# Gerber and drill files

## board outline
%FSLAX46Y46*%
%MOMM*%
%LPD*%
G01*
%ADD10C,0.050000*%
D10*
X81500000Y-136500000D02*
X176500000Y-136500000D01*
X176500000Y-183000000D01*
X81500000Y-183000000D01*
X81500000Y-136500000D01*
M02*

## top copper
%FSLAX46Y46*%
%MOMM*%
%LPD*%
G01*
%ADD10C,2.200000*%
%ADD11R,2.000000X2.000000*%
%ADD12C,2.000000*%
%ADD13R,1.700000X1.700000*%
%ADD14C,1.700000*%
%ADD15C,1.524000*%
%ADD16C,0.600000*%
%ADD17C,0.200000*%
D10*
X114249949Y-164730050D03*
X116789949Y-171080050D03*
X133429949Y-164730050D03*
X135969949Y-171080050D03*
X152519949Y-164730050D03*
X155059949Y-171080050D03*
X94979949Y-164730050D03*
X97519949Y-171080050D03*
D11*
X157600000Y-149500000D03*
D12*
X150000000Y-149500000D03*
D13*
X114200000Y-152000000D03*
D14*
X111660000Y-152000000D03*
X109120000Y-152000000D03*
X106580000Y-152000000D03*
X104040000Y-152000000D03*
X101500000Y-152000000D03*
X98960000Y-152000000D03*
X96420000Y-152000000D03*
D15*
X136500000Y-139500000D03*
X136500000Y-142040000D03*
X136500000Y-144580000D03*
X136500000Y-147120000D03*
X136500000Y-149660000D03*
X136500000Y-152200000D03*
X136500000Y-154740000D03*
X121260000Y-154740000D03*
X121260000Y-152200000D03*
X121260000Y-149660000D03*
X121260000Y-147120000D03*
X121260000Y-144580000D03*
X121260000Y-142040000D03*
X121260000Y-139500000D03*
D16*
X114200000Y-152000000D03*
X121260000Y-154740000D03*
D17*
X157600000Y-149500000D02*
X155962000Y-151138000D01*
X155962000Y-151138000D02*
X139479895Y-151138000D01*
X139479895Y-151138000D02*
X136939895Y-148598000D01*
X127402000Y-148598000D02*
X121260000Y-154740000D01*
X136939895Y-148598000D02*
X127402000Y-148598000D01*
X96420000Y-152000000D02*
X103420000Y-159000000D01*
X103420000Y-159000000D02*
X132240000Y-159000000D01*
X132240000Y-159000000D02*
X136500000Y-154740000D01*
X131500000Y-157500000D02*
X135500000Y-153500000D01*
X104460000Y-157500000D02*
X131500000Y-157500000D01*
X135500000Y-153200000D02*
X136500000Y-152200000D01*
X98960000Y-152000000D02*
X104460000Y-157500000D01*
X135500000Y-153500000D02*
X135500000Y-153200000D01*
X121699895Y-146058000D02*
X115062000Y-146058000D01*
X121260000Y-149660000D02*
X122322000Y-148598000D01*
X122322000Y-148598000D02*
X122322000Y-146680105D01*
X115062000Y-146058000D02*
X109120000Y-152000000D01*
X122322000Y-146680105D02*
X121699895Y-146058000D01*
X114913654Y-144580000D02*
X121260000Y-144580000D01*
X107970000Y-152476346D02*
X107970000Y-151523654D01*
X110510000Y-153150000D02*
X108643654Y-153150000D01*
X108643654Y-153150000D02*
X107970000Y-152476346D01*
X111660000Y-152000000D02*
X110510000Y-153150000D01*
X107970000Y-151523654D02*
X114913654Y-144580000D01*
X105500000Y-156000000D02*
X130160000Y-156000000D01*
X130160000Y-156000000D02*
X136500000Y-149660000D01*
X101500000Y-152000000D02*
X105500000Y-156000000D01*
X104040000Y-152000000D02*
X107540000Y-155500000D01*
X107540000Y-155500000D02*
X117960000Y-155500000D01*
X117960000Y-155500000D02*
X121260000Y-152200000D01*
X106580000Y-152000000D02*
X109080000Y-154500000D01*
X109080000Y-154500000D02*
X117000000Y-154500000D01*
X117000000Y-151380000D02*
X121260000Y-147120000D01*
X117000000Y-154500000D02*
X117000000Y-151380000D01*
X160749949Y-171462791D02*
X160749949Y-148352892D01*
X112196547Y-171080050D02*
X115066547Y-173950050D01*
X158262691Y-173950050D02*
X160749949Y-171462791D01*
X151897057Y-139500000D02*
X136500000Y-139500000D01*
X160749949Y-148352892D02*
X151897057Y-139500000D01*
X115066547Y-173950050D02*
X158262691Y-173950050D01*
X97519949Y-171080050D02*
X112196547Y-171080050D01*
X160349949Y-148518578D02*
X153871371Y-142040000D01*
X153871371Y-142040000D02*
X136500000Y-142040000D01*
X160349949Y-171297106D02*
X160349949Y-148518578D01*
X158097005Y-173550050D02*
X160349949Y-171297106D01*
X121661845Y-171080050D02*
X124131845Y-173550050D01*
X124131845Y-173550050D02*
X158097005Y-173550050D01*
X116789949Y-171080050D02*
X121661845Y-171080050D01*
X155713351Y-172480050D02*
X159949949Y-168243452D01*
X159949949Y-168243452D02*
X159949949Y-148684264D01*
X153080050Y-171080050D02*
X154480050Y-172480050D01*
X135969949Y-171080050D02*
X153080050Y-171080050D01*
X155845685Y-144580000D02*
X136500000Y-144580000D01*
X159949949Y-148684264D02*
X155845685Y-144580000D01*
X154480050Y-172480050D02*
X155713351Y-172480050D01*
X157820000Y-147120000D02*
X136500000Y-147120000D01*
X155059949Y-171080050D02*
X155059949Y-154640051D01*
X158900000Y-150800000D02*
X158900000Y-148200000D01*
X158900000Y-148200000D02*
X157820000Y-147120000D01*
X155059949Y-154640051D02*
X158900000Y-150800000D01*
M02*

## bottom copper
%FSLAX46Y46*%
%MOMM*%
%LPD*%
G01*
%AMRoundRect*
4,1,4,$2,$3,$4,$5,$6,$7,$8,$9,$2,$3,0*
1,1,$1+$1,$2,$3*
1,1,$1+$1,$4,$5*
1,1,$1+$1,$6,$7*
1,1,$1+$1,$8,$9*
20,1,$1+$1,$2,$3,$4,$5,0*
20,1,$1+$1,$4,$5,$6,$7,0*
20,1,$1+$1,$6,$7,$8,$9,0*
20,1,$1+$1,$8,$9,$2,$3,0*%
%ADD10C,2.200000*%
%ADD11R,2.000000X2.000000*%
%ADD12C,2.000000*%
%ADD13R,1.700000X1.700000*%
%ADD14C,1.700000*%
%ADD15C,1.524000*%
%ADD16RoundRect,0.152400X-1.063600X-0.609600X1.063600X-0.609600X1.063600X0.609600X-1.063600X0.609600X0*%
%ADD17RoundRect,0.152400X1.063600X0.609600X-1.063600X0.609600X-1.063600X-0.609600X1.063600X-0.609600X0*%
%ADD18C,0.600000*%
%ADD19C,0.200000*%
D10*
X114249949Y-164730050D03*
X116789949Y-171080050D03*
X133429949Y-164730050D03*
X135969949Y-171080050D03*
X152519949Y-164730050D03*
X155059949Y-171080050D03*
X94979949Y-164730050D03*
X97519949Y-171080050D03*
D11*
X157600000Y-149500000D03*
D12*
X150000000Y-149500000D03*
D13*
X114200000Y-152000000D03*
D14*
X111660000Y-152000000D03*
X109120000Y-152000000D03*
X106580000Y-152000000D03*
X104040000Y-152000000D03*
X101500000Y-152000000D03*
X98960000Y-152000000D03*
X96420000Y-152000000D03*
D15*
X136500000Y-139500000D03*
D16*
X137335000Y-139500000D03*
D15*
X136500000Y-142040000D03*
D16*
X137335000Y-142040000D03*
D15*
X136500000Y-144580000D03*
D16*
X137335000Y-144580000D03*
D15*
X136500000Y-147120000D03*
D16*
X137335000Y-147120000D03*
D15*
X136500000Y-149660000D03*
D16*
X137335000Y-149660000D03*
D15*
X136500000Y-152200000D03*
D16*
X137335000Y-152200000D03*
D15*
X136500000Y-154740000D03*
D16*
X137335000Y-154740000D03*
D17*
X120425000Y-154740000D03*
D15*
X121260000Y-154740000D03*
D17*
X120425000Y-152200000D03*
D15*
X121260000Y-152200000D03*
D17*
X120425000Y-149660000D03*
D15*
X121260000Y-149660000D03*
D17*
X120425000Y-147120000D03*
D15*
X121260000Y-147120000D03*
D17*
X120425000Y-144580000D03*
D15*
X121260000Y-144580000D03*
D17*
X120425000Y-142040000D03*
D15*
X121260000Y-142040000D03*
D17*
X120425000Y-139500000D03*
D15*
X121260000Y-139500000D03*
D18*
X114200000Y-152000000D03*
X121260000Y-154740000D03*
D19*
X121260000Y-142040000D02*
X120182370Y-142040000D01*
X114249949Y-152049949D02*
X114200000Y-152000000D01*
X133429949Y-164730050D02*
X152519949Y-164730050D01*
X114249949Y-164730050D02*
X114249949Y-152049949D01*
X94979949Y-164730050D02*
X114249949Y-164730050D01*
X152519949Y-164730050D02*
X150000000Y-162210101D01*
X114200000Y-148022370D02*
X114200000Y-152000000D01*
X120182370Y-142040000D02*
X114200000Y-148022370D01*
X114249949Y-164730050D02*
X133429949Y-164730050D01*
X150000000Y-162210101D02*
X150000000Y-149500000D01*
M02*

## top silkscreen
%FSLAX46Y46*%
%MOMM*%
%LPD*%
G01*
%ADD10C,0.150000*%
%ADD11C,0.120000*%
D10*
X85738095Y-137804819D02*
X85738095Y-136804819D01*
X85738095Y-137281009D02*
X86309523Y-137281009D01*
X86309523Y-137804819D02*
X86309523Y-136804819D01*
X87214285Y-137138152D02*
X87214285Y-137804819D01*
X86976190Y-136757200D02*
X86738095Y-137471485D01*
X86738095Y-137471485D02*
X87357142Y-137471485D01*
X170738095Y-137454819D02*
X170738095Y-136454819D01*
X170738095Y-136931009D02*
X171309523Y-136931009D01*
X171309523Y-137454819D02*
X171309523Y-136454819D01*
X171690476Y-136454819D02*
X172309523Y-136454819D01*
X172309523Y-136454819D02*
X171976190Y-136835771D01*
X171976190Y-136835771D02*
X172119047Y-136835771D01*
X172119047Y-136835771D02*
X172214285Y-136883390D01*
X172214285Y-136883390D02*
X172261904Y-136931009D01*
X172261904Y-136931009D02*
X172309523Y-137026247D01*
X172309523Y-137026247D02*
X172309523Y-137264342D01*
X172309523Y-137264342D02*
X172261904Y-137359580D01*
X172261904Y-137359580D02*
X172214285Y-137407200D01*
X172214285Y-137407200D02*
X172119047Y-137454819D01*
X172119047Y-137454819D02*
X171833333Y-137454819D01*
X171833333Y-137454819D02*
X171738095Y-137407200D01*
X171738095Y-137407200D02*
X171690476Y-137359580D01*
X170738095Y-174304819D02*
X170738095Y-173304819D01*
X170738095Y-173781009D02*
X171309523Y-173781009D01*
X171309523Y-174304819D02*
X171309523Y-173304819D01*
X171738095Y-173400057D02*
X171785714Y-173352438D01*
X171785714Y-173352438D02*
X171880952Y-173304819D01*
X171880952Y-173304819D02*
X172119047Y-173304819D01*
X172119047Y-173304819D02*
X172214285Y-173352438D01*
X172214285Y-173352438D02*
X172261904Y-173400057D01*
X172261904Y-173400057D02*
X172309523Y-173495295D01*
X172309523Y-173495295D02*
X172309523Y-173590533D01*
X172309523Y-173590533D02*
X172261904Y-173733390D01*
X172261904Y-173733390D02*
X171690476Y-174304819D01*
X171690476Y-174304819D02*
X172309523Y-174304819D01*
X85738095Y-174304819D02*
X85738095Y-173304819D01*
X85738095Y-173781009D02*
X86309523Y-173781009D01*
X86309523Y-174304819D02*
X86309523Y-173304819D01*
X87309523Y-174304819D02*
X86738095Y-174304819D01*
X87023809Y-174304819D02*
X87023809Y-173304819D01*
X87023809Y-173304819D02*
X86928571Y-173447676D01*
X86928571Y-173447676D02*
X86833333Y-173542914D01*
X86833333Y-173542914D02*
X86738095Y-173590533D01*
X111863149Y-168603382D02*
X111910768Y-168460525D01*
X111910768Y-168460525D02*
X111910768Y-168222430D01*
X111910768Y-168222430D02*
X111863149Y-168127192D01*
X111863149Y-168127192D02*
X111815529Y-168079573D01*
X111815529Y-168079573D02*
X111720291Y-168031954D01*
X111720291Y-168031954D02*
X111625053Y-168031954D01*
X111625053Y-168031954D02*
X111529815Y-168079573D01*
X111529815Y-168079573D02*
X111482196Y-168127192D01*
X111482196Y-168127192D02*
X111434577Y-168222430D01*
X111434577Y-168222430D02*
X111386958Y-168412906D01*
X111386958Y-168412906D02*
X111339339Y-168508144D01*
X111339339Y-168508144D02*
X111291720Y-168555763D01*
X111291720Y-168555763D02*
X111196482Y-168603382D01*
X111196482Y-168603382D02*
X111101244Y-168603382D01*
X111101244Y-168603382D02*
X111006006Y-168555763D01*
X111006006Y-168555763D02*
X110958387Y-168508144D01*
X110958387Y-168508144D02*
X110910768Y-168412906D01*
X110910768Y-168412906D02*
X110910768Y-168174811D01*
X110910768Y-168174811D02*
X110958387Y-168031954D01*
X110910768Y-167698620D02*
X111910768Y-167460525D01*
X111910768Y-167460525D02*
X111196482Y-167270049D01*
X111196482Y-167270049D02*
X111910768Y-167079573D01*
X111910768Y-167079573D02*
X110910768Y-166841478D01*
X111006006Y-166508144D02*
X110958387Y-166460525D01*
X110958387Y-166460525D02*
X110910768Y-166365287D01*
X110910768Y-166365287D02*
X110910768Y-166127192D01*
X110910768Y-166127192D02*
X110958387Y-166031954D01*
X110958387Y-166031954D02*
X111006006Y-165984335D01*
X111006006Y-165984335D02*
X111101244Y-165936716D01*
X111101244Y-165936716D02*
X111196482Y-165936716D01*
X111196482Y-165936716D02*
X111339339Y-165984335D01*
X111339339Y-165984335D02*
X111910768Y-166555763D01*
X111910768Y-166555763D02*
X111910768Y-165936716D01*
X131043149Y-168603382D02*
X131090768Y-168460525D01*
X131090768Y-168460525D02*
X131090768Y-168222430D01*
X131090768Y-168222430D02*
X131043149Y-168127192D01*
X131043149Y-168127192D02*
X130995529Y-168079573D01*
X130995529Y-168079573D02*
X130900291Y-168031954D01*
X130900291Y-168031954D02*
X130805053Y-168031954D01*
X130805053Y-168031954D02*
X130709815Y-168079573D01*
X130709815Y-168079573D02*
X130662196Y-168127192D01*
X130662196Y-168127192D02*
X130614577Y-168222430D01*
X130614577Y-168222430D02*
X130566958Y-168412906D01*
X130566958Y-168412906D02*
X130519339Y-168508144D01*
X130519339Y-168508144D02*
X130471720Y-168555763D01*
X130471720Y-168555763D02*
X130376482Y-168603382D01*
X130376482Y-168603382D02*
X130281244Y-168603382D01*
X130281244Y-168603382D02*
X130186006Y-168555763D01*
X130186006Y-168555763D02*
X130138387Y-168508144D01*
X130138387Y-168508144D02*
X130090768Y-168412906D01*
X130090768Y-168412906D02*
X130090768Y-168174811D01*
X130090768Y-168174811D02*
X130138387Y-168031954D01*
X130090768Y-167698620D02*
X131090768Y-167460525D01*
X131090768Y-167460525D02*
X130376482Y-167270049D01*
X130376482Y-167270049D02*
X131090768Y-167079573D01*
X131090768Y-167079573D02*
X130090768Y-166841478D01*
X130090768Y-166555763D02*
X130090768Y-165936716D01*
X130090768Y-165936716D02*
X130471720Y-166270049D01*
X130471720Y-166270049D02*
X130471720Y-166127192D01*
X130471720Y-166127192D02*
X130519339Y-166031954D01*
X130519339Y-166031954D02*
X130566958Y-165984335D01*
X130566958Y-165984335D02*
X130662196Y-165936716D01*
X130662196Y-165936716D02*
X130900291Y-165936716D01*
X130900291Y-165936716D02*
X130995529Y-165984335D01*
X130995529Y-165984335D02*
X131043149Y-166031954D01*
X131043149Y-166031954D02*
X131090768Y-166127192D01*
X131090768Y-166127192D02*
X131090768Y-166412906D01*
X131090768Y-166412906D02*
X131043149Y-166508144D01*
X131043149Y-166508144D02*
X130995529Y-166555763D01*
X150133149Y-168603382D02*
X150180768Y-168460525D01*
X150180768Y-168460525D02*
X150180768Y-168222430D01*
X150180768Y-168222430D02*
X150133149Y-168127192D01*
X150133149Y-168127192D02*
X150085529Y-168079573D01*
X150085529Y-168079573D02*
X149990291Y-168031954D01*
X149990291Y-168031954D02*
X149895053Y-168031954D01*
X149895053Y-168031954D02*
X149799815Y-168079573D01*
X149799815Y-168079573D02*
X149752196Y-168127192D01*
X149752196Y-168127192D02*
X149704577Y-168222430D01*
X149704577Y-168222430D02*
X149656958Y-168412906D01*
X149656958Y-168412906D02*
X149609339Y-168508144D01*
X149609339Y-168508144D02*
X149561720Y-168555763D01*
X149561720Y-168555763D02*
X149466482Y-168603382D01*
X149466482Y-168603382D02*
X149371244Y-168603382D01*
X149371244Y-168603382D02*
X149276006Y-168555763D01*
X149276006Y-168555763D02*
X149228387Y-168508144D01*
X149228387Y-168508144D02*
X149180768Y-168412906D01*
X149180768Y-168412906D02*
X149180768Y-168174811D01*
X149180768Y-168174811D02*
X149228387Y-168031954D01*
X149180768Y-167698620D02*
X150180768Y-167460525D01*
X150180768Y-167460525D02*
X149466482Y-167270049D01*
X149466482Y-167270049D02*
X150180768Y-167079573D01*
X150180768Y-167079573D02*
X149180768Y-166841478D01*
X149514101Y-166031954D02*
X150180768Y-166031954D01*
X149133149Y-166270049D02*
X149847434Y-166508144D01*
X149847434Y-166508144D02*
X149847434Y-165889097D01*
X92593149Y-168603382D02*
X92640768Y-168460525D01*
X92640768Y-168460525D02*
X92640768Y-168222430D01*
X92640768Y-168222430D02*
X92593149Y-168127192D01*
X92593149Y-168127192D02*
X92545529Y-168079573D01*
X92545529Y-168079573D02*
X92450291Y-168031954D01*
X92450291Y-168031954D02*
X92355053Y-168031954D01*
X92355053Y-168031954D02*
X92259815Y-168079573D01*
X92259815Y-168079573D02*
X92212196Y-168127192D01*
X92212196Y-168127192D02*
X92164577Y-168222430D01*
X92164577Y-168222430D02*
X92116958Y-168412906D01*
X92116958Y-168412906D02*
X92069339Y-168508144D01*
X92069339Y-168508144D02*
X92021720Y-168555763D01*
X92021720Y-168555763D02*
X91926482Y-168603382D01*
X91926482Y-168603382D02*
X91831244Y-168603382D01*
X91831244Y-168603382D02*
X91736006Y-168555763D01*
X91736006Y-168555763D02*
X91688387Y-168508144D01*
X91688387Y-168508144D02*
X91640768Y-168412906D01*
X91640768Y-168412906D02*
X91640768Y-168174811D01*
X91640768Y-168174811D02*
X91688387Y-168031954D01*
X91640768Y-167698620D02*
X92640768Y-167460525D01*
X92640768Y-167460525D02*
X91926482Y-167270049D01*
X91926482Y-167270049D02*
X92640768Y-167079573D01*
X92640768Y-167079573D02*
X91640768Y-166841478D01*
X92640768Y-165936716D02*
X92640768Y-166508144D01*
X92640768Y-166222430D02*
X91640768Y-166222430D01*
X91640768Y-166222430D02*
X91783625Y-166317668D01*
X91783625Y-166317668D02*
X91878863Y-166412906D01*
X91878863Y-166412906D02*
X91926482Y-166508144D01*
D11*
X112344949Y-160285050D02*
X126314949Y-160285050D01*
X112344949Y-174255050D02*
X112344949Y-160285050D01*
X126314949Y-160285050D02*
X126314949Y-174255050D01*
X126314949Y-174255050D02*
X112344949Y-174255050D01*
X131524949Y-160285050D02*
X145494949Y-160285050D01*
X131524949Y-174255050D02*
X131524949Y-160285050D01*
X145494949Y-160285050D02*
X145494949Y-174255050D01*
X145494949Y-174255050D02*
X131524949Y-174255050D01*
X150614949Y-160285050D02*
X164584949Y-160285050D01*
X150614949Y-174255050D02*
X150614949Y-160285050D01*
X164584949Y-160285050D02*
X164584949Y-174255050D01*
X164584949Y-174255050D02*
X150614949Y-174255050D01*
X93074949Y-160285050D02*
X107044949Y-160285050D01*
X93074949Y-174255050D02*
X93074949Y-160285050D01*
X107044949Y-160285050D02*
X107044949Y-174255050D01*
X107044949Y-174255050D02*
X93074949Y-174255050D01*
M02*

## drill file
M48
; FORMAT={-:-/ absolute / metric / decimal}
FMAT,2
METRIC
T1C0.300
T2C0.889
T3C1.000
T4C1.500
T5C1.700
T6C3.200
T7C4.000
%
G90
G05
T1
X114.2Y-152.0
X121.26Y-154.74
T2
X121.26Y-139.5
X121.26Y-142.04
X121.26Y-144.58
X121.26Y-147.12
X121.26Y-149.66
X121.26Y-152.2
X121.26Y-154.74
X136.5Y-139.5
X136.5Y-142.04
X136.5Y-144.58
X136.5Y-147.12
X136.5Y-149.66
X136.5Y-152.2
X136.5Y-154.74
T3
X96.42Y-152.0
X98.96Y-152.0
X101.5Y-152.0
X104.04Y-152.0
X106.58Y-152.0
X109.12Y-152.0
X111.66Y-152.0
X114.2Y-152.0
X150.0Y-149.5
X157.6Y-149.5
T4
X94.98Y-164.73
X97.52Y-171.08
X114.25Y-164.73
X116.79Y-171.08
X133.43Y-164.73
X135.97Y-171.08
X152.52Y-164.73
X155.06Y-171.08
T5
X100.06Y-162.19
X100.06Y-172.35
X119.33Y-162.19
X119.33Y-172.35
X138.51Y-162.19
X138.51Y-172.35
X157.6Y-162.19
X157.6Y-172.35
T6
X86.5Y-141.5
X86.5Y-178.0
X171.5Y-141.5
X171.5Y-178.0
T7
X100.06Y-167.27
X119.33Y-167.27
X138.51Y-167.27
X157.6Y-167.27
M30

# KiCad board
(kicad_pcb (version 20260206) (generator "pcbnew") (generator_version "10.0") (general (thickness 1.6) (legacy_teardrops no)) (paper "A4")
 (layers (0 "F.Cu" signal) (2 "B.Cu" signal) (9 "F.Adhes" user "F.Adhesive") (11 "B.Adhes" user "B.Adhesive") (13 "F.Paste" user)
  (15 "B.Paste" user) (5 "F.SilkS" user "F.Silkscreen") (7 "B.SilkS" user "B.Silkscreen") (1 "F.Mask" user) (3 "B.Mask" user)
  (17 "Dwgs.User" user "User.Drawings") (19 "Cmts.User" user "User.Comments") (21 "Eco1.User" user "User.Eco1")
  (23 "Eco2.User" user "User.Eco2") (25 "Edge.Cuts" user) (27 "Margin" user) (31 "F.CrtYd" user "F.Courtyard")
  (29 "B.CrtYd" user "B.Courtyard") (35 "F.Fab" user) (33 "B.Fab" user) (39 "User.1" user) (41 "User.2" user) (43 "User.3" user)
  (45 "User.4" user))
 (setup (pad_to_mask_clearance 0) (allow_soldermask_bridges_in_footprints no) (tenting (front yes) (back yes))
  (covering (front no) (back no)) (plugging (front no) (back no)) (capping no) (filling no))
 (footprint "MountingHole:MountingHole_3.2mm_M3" (layer "F.Cu") (at 86.5 141.5)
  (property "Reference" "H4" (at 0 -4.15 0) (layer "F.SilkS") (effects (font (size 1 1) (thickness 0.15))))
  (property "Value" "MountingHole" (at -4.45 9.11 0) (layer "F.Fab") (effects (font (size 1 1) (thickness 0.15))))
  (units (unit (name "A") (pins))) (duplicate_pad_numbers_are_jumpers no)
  (pad "" np_thru_hole circle (at 0 0) (size 3.2 3.2) (drill 3.2) (layers "*.Cu" "*.Mask")))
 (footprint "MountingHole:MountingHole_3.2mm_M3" (layer "F.Cu") (at 171.5 141.5)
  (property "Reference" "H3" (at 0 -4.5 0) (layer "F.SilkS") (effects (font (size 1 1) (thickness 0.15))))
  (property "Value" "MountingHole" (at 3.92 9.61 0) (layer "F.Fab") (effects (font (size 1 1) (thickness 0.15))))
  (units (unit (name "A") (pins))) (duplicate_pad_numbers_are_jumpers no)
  (pad "" np_thru_hole circle (at 0 0) (size 3.2 3.2) (drill 3.2) (layers "*.Cu" "*.Mask")))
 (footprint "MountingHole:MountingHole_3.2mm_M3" (layer "F.Cu") (at 171.5 178)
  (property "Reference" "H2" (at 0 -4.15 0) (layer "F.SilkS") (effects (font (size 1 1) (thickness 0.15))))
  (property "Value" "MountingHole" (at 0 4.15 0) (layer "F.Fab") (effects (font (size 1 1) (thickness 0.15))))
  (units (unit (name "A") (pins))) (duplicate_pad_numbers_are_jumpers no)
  (pad "" np_thru_hole circle (at 0 0) (size 3.2 3.2) (drill 3.2) (layers "*.Cu" "*.Mask")))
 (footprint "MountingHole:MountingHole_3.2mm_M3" (layer "F.Cu") (at 86.5 178)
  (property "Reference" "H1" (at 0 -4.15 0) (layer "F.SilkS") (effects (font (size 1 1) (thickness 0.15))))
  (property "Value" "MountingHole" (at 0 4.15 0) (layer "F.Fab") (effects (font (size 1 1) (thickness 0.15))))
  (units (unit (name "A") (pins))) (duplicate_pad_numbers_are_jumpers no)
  (pad "" np_thru_hole circle (at 0 0) (size 3.2 3.2) (drill 3.2) (layers "*.Cu" "*.Mask")))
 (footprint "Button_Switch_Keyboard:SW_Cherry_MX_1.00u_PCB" (layer "F.Cu") (at 114.249949 164.73005 90)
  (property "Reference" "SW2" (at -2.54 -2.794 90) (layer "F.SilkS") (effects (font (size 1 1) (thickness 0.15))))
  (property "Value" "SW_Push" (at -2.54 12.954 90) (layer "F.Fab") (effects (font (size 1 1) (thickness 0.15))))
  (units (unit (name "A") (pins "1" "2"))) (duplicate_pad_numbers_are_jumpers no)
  (fp_line (start 4.445 -1.905) (end 4.445 12.065) (stroke (width 0.12) (type solid)) (layer "F.SilkS"))
  (fp_line (start -9.525 -1.905) (end 4.445 -1.905) (stroke (width 0.12) (type solid)) (layer "F.SilkS"))
  (fp_line (start 4.445 12.065) (end -9.525 12.065) (stroke (width 0.12) (type solid)) (layer "F.SilkS"))
  (fp_line (start -9.525 12.065) (end -9.525 -1.905) (stroke (width 0.12) (type solid)) (layer "F.SilkS"))
  (pad "" np_thru_hole circle (at -7.62 5.08 90) (size 1.7 1.7) (drill 1.7) (layers "*.Cu" "*.Mask"))
  (pad "" np_thru_hole circle (at -2.54 5.08 90) (size 4 4) (drill 4) (layers "*.Cu" "*.Mask"))
  (pad "" np_thru_hole circle (at 2.54 5.08 90) (size 1.7 1.7) (drill 1.7) (layers "*.Cu" "*.Mask"))
  (pad "1" thru_hole circle (at 0 0 90) (size 2.2 2.2) (drill 1.5) (layers "*.Cu" "*.Mask") (remove_unused_layers no) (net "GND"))
  (pad "2" thru_hole circle (at -6.35 2.54 90) (size 2.2 2.2) (drill 1.5) (layers "*.Cu" "*.Mask") (remove_unused_layers no)
   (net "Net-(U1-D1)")))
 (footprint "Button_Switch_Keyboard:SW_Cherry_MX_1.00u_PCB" (layer "F.Cu") (at 133.429949 164.73005 90)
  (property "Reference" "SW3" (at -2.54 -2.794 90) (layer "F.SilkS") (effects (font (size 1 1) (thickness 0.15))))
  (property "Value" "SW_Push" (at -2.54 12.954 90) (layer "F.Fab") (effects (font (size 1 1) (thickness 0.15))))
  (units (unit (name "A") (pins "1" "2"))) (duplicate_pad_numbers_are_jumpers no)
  (fp_line (start 4.445 -1.905) (end 4.445 12.065) (stroke (width 0.12) (type solid)) (layer "F.SilkS"))
  (fp_line (start -9.525 -1.905) (end 4.445 -1.905) (stroke (width 0.12) (type solid)) (layer "F.SilkS"))
  (fp_line (start 4.445 12.065) (end -9.525 12.065) (stroke (width 0.12) (type solid)) (layer "F.SilkS"))
  (fp_line (start -9.525 12.065) (end -9.525 -1.905) (stroke (width 0.12) (type solid)) (layer "F.SilkS"))
  (pad "" np_thru_hole circle (at -7.62 5.08 90) (size 1.7 1.7) (drill 1.7) (layers "*.Cu" "*.Mask"))
  (pad "" np_thru_hole circle (at -2.54 5.08 90) (size 4 4) (drill 4) (layers "*.Cu" "*.Mask"))
  (pad "" np_thru_hole circle (at 2.54 5.08 90) (size 1.7 1.7) (drill 1.7) (layers "*.Cu" "*.Mask"))
  (pad "1" thru_hole circle (at 0 0 90) (size 2.2 2.2) (drill 1.5) (layers "*.Cu" "*.Mask") (remove_unused_layers no) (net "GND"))
  (pad "2" thru_hole circle (at -6.35 2.54 90) (size 2.2 2.2) (drill 1.5) (layers "*.Cu" "*.Mask") (remove_unused_layers no)
   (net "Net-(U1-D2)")))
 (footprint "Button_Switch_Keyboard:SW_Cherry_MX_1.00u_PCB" (layer "F.Cu") (at 152.519949 164.73005 90)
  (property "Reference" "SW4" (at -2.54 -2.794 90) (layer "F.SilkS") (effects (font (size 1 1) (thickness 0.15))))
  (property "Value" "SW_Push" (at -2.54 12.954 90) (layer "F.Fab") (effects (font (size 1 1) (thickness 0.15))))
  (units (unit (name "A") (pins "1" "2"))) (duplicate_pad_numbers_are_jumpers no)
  (fp_line (start 4.445 -1.905) (end 4.445 12.065) (stroke (width 0.12) (type solid)) (layer "F.SilkS"))
  (fp_line (start -9.525 -1.905) (end 4.445 -1.905) (stroke (width 0.12) (type solid)) (layer "F.SilkS"))
  (fp_line (start 4.445 12.065) (end -9.525 12.065) (stroke (width 0.12) (type solid)) (layer "F.SilkS"))
  (fp_line (start -9.525 12.065) (end -9.525 -1.905) (stroke (width 0.12) (type solid)) (layer "F.SilkS"))
  (pad "" np_thru_hole circle (at -7.62 5.08 90) (size 1.7 1.7) (drill 1.7) (layers "*.Cu" "*.Mask"))
  (pad "" np_thru_hole circle (at -2.54 5.08 90) (size 4 4) (drill 4) (layers "*.Cu" "*.Mask"))
  (pad "" np_thru_hole circle (at 2.54 5.08 90) (size 1.7 1.7) (drill 1.7) (layers "*.Cu" "*.Mask"))
  (pad "1" thru_hole circle (at 0 0 90) (size 2.2 2.2) (drill 1.5) (layers "*.Cu" "*.Mask") (remove_unused_layers no) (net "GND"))
  (pad "2" thru_hole circle (at -6.35 2.54 90) (size 2.2 2.2) (drill 1.5) (layers "*.Cu" "*.Mask") (remove_unused_layers no)
   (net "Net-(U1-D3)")))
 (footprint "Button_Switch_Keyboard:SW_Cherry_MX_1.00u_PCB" (layer "F.Cu") (at 94.979949 164.73005 90)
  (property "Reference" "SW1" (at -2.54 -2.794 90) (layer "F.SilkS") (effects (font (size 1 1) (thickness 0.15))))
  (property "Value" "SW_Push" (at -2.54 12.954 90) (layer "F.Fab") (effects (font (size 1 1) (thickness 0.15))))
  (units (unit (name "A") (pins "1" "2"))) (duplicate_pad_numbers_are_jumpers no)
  (fp_line (start 4.445 -1.905) (end 4.445 12.065) (stroke (width 0.12) (type solid)) (layer "F.SilkS"))
  (fp_line (start -9.525 -1.905) (end 4.445 -1.905) (stroke (width 0.12) (type solid)) (layer "F.SilkS"))
  (fp_line (start 4.445 12.065) (end -9.525 12.065) (stroke (width 0.12) (type solid)) (layer "F.SilkS"))
  (fp_line (start -9.525 12.065) (end -9.525 -1.905) (stroke (width 0.12) (type solid)) (layer "F.SilkS"))
  (pad "" np_thru_hole circle (at -7.62 5.08 90) (size 1.7 1.7) (drill 1.7) (layers "*.Cu" "*.Mask"))
  (pad "" np_thru_hole circle (at -2.54 5.08 90) (size 4 4) (drill 4) (layers "*.Cu" "*.Mask"))
  (pad "" np_thru_hole circle (at 2.54 5.08 90) (size 1.7 1.7) (drill 1.7) (layers "*.Cu" "*.Mask"))
  (pad "1" thru_hole circle (at 0 0 90) (size 2.2 2.2) (drill 1.5) (layers "*.Cu" "*.Mask") (remove_unused_layers no) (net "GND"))
  (pad "2" thru_hole circle (at -6.35 2.54 90) (size 2.2 2.2) (drill 1.5) (layers "*.Cu" "*.Mask") (remove_unused_layers no)
   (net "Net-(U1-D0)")))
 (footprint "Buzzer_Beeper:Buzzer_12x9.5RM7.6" (layer "B.Cu") (at 157.6 149.5 180)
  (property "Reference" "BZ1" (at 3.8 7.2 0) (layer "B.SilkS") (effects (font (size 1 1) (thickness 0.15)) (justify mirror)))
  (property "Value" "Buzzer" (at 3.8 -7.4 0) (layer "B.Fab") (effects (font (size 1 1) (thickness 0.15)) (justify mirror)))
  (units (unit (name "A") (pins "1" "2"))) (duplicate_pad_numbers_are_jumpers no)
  (pad "1" thru_hole rect (at 0 0 180) (size 2 2) (drill 1) (layers "*.Cu" "*.Mask") (remove_unused_layers no) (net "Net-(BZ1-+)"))
  (pad "2" thru_hole circle (at 7.6 0 180) (size 2 2) (drill 1) (layers "*.Cu" "*.Mask") (remove_unused_layers no) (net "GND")))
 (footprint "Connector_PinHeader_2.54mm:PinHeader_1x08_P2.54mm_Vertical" (layer "B.Cu") (at 114.2 152 90)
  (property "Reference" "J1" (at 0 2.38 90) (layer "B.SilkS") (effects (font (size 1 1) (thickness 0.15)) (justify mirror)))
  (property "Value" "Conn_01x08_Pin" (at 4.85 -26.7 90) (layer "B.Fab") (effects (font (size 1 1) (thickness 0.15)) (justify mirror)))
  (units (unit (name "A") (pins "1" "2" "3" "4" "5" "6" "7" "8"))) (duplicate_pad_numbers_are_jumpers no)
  (pad "1" thru_hole rect (at 0 0 90) (size 1.7 1.7) (drill 1) (layers "*.Cu" "*.Mask") (remove_unused_layers no) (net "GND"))
  (pad "2" thru_hole circle (at 0 -2.54 90) (size 1.7 1.7) (drill 1) (layers "*.Cu" "*.Mask") (remove_unused_layers no) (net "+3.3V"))
  (pad "3" thru_hole circle (at 0 -5.08 90) (size 1.7 1.7) (drill 1) (layers "*.Cu" "*.Mask") (remove_unused_layers no) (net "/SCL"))
  (pad "4" thru_hole circle (at 0 -7.62 90) (size 1.7 1.7) (drill 1) (layers "*.Cu" "*.Mask") (remove_unused_layers no) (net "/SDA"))
  (pad "5" thru_hole circle (at 0 -10.16 90) (size 1.7 1.7) (drill 1) (layers "*.Cu" "*.Mask") (remove_unused_layers no) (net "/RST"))
  (pad "6" thru_hole circle (at 0 -12.7 90) (size 1.7 1.7) (drill 1) (layers "*.Cu" "*.Mask") (remove_unused_layers no) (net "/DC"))
  (pad "7" thru_hole circle (at 0 -15.24 90) (size 1.7 1.7) (drill 1) (layers "*.Cu" "*.Mask") (remove_unused_layers no) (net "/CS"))
  (pad "8" thru_hole circle (at 0 -17.78 90) (size 1.7 1.7) (drill 1) (layers "*.Cu" "*.Mask") (remove_unused_layers no) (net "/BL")))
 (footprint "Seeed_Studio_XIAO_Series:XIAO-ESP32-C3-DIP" (layer "B.Cu") (at 128.88 147.12 90)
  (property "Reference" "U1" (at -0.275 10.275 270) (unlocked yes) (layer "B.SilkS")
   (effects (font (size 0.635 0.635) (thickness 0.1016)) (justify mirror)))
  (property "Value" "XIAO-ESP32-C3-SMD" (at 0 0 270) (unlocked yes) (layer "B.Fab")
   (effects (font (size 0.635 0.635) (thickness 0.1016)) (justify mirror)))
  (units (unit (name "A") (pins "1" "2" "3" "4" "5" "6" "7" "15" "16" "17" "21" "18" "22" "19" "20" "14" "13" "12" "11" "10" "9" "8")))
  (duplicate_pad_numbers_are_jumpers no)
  (pad "1" thru_hole circle (at 7.62 7.62) (size 1.524 1.524) (drill 0.889) (layers "*.Cu" "*.Mask") (remove_unused_layers no)
   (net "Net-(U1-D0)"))
  (pad "1" smd roundrect (at 7.62 8.455) (size 2.432 1.524) (layers "B.Cu" "B.Mask") (roundrect_rratio 0.1) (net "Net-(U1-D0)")
   (thermal_bridge_angle 45))
  (pad "2" thru_hole circle (at 5.08 7.62) (size 1.524 1.524) (drill 0.889) (layers "*.Cu" "*.Mask") (remove_unused_layers no)
   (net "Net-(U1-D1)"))
  (pad "2" smd roundrect (at 5.08 8.455) (size 2.432 1.524) (layers "B.Cu" "B.Mask") (roundrect_rratio 0.1) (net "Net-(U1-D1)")
   (thermal_bridge_angle 45))
  (pad "3" thru_hole circle (at 2.54 7.62) (size 1.524 1.524) (drill 0.889) (layers "*.Cu" "*.Mask") (remove_unused_layers no)
   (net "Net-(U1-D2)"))
  (pad "3" smd roundrect (at 2.54 8.455) (size 2.432 1.524) (layers "B.Cu" "B.Mask") (roundrect_rratio 0.1) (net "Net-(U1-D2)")
   (thermal_bridge_angle 45))
  (pad "4" thru_hole circle (at 0 7.62) (size 1.524 1.524) (drill 0.889) (layers "*.Cu" "*.Mask") (remove_unused_layers no)
   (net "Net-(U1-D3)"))
  (pad "4" smd roundrect (at 0 8.455) (size 2.432 1.524) (layers "B.Cu" "B.Mask") (roundrect_rratio 0.1) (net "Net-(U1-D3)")
   (thermal_bridge_angle 45))
  (pad "5" thru_hole circle (at -2.54 7.62) (size 1.524 1.524) (drill 0.889) (layers "*.Cu" "*.Mask") (remove_unused_layers no) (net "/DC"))
  (pad "5" smd roundrect (at -2.54 8.455) (size 2.432 1.524) (layers "B.Cu" "B.Mask") (roundrect_rratio 0.1) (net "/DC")
   (thermal_bridge_angle 45))
  (pad "6" thru_hole circle (at -5.08 7.62) (size 1.524 1.524) (drill 0.889) (layers "*.Cu" "*.Mask") (remove_unused_layers no) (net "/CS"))
  (pad "6" smd roundrect (at -5.08 8.455) (size 2.432 1.524) (layers "B.Cu" "B.Mask") (roundrect_rratio 0.1) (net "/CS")
   (thermal_bridge_angle 45))
  (pad "7" thru_hole circle (at -7.62 7.62) (size 1.524 1.524) (drill 0.889) (layers "*.Cu" "*.Mask") (remove_unused_layers no) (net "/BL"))
  (pad "7" smd roundrect (at -7.62 8.455) (size 2.432 1.524) (layers "B.Cu" "B.Mask") (roundrect_rratio 0.1) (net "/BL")
   (thermal_bridge_angle 45))
  (pad "8" smd roundrect (at -7.62 -8.455 180) (size 2.432 1.524) (layers "B.Cu" "B.Mask") (roundrect_rratio 0.1) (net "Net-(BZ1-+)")
   (thermal_bridge_angle 45))
  (pad "8" thru_hole circle (at -7.62 -7.62 180) (size 1.524 1.524) (drill 0.889) (layers "*.Cu" "*.Mask") (remove_unused_layers no)
   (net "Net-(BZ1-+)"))
  (pad "9" smd roundrect (at -5.08 -8.455 180) (size 2.432 1.524) (layers "B.Cu" "B.Mask") (roundrect_rratio 0.1) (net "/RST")
   (thermal_bridge_angle 45))
  (pad "9" thru_hole circle (at -5.08 -7.62 180) (size 1.524 1.524) (drill 0.889) (layers "*.Cu" "*.Mask") (remove_unused_layers no)
   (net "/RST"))
  (pad "10" smd roundrect (at -2.54 -8.455 180) (size 2.432 1.524) (layers "B.Cu" "B.Mask") (roundrect_rratio 0.1) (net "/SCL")
   (thermal_bridge_angle 45))
  (pad "10" thru_hole circle (at -2.54 -7.62 180) (size 1.524 1.524) (drill 0.889) (layers "*.Cu" "*.Mask") (remove_unused_layers no)
   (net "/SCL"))
  (pad "11" smd roundrect (at 0 -8.455 180) (size 2.432 1.524) (layers "B.Cu" "B.Mask") (roundrect_rratio 0.1) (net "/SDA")
   (thermal_bridge_angle 45))
  (pad "11" thru_hole circle (at 0 -7.62 180) (size 1.524 1.524) (drill 0.889) (layers "*.Cu" "*.Mask") (remove_unused_layers no)
   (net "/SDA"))
  (pad "12" smd roundrect (at 2.54 -8.455 180) (size 2.432 1.524) (layers "B.Cu" "B.Mask") (roundrect_rratio 0.1) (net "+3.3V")
   (thermal_bridge_angle 45))
  (pad "12" thru_hole circle (at 2.54 -7.62 180) (size 1.524 1.524) (drill 0.889) (layers "*.Cu" "*.Mask") (remove_unused_layers no)
   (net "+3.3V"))
  (pad "13" smd roundrect (at 5.08 -8.455 180) (size 2.432 1.524) (layers "B.Cu" "B.Mask") (roundrect_rratio 0.1) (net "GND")
   (thermal_bridge_angle 45))
  (pad "13" thru_hole circle (at 5.08 -7.62 180) (size 1.524 1.524) (drill 0.889) (layers "*.Cu" "*.Mask") (remove_unused_layers no)
   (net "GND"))
  (pad "14" smd roundrect (at 7.62 -8.455 180) (size 2.432 1.524) (layers "B.Cu" "B.Mask") (roundrect_rratio 0.1)
   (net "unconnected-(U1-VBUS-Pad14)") (thermal_bridge_angle 45))
  (pad "14" thru_hole circle (at 7.62 -7.62 180) (size 1.524 1.524) (drill 0.889) (layers "*.Cu" "*.Mask") (remove_unused_layers no)
   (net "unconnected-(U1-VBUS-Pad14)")))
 (gr_rect (start 81.5 136.5) (end 176.5 183) (stroke (width 0.05) (type default)) (fill no) (layer "Edge.Cuts"))
 (via (at 114.2 152) (size 0.6) (drill 0.3) (layers "F.Cu" "B.Cu") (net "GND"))
 (segment (start 121.26 142.04) (end 120.18237 142.04) (width 0.2) (layer "B.Cu") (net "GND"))
 (segment (start 114.249949 152.049949) (end 114.2 152) (width 0.2) (layer "B.Cu") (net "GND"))
 (segment (start 133.429949 164.73005) (end 152.519949 164.73005) (width 0.2) (layer "B.Cu") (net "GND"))
 (segment (start 114.249949 164.73005) (end 114.249949 152.049949) (width 0.2) (layer "B.Cu") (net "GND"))
 (segment (start 94.979949 164.73005) (end 114.249949 164.73005) (width 0.2) (layer "B.Cu") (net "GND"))
 (segment (start 152.519949 164.73005) (end 150 162.210101) (width 0.2) (layer "B.Cu") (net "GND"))
 (segment (start 114.2 148.02237) (end 114.2 152) (width 0.2) (layer "B.Cu") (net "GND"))
 (segment (start 120.18237 142.04) (end 114.2 148.02237) (width 0.2) (layer "B.Cu") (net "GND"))
 (segment (start 114.249949 164.73005) (end 133.429949 164.73005) (width 0.2) (layer "B.Cu") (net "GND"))
 (segment (start 150 162.210101) (end 150 149.5) (width 0.2) (layer "B.Cu") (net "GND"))
 (segment (start 157.6 149.5) (end 155.962 151.138) (width 0.2) (layer "F.Cu") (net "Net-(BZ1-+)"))
 (segment (start 155.962 151.138) (end 139.479895 151.138) (width 0.2) (layer "F.Cu") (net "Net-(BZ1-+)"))
 (segment (start 139.479895 151.138) (end 136.939895 148.598) (width 0.2) (layer "F.Cu") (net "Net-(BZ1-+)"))
 (segment (start 127.402 148.598) (end 121.26 154.74) (width 0.2) (layer "F.Cu") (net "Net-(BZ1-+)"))
 (segment (start 136.939895 148.598) (end 127.402 148.598) (width 0.2) (layer "F.Cu") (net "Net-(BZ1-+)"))
 (via (at 121.26 154.74) (size 0.6) (drill 0.3) (layers "F.Cu" "B.Cu") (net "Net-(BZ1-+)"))
 (segment (start 96.42 152) (end 103.42 159) (width 0.2) (layer "F.Cu") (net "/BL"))
 (segment (start 103.42 159) (end 132.24 159) (width 0.2) (layer "F.Cu") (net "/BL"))
 (segment (start 132.24 159) (end 136.5 154.74) (width 0.2) (layer "F.Cu") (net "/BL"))
 (segment (start 131.5 157.5) (end 135.5 153.5) (width 0.2) (layer "F.Cu") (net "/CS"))
 (segment (start 104.46 157.5) (end 131.5 157.5) (width 0.2) (layer "F.Cu") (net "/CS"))
 (segment (start 135.5 153.2) (end 136.5 152.2) (width 0.2) (layer "F.Cu") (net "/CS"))
 (segment (start 98.96 152) (end 104.46 157.5) (width 0.2) (layer "F.Cu") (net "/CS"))
 (segment (start 135.5 153.5) (end 135.5 153.2) (width 0.2) (layer "F.Cu") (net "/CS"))
 (segment (start 121.699895 146.058) (end 115.062 146.058) (width 0.2) (layer "F.Cu") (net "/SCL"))
 (segment (start 121.26 149.66) (end 122.322 148.598) (width 0.2) (layer "F.Cu") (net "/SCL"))
 (segment (start 122.322 148.598) (end 122.322 146.680105) (width 0.2) (layer "F.Cu") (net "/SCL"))
 (segment (start 115.062 146.058) (end 109.12 152) (width 0.2) (layer "F.Cu") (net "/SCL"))
 (segment (start 122.322 146.680105) (end 121.699895 146.058) (width 0.2) (layer "F.Cu") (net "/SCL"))
 (segment (start 114.913654 144.58) (end 121.26 144.58) (width 0.2) (layer "F.Cu") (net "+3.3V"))
 (segment (start 107.97 152.476346) (end 107.97 151.523654) (width 0.2) (layer "F.Cu") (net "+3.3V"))
 (segment (start 110.51 153.15) (end 108.643654 153.15) (width 0.2) (layer "F.Cu") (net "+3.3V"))
 (segment (start 108.643654 153.15) (end 107.97 152.476346) (width 0.2) (layer "F.Cu") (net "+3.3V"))
 (segment (start 111.66 152) (end 110.51 153.15) (width 0.2) (layer "F.Cu") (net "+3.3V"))
 (segment (start 107.97 151.523654) (end 114.913654 144.58) (width 0.2) (layer "F.Cu") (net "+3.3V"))
 (segment (start 105.5 156) (end 130.16 156) (width 0.2) (layer "F.Cu") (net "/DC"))
 (segment (start 130.16 156) (end 136.5 149.66) (width 0.2) (layer "F.Cu") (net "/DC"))
 (segment (start 101.5 152) (end 105.5 156) (width 0.2) (layer "F.Cu") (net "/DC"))
 (segment (start 104.04 152) (end 107.54 155.5) (width 0.2) (layer "F.Cu") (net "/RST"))
 (segment (start 107.54 155.5) (end 117.96 155.5) (width 0.2) (layer "F.Cu") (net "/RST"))
 (segment (start 117.96 155.5) (end 121.26 152.2) (width 0.2) (layer "F.Cu") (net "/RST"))
 (segment (start 106.58 152) (end 109.08 154.5) (width 0.2) (layer "F.Cu") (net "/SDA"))
 (segment (start 109.08 154.5) (end 117 154.5) (width 0.2) (layer "F.Cu") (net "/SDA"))
 (segment (start 117 151.38) (end 121.26 147.12) (width 0.2) (layer "F.Cu") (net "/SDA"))
 (segment (start 117 154.5) (end 117 151.38) (width 0.2) (layer "F.Cu") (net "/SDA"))
 (segment (start 160.749949 171.462791) (end 160.749949 148.352892) (width 0.2) (layer "F.Cu") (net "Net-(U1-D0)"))
 (segment (start 112.196547 171.08005) (end 115.066547 173.95005) (width 0.2) (layer "F.Cu") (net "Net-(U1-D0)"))
 (segment (start 158.262691 173.95005) (end 160.749949 171.462791) (width 0.2) (layer "F.Cu") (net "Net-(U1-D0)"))
 (segment (start 151.897057 139.5) (end 136.5 139.5) (width 0.2) (layer "F.Cu") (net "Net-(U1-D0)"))
 (segment (start 160.749949 148.352892) (end 151.897057 139.5) (width 0.2) (layer "F.Cu") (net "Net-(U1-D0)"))
 (segment (start 115.066547 173.95005) (end 158.262691 173.95005) (width 0.2) (layer "F.Cu") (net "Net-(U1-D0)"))
 (segment (start 97.519949 171.08005) (end 112.196547 171.08005) (width 0.2) (layer "F.Cu") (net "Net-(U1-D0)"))
 (segment (start 160.349949 148.518578) (end 153.871371 142.04) (width 0.2) (layer "F.Cu") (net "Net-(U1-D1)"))
 (segment (start 153.871371 142.04) (end 136.5 142.04) (width 0.2) (layer "F.Cu") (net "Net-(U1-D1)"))
 (segment (start 160.349949 171.297106) (end 160.349949 148.518578) (width 0.2) (layer "F.Cu") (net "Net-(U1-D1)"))
 (segment (start 158.097005 173.55005) (end 160.349949 171.297106) (width 0.2) (layer "F.Cu") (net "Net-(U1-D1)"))
 (segment (start 121.661845 171.08005) (end 124.131845 173.55005) (width 0.2) (layer "F.Cu") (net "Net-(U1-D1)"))
 (segment (start 124.131845 173.55005) (end 158.097005 173.55005) (width 0.2) (layer "F.Cu") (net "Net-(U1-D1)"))
 (segment (start 116.789949 171.08005) (end 121.661845 171.08005) (width 0.2) (layer "F.Cu") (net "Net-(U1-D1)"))
 (segment (start 155.713351 172.48005) (end 159.949949 168.243452) (width 0.2) (layer "F.Cu") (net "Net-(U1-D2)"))
 (segment (start 159.949949 168.243452) (end 159.949949 148.684264) (width 0.2) (layer "F.Cu") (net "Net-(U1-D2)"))
 (segment (start 153.08005 171.08005) (end 154.48005 172.48005) (width 0.2) (layer "F.Cu") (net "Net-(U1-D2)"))
 (segment (start 135.969949 171.08005) (end 153.08005 171.08005) (width 0.2) (layer "F.Cu") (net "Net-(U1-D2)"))
 (segment (start 155.845685 144.58) (end 136.5 144.58) (width 0.2) (layer "F.Cu") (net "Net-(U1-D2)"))
 (segment (start 159.949949 148.684264) (end 155.845685 144.58) (width 0.2) (layer "F.Cu") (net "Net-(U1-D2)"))
 (segment (start 154.48005 172.48005) (end 155.713351 172.48005) (width 0.2) (layer "F.Cu") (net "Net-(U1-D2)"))
 (segment (start 157.82 147.12) (end 136.5 147.12) (width 0.2) (layer "F.Cu") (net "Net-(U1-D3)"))
 (segment (start 155.059949 171.08005) (end 155.059949 154.640051) (width 0.2) (layer "F.Cu") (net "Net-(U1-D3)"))
 (segment (start 158.9 150.8) (end 158.9 148.2) (width 0.2) (layer "F.Cu") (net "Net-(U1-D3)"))
 (segment (start 158.9 148.2) (end 157.82 147.12) (width 0.2) (layer "F.Cu") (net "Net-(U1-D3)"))
 (segment (start 155.059949 154.640051) (end 158.9 150.8) (width 0.2) (layer "F.Cu") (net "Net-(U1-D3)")))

